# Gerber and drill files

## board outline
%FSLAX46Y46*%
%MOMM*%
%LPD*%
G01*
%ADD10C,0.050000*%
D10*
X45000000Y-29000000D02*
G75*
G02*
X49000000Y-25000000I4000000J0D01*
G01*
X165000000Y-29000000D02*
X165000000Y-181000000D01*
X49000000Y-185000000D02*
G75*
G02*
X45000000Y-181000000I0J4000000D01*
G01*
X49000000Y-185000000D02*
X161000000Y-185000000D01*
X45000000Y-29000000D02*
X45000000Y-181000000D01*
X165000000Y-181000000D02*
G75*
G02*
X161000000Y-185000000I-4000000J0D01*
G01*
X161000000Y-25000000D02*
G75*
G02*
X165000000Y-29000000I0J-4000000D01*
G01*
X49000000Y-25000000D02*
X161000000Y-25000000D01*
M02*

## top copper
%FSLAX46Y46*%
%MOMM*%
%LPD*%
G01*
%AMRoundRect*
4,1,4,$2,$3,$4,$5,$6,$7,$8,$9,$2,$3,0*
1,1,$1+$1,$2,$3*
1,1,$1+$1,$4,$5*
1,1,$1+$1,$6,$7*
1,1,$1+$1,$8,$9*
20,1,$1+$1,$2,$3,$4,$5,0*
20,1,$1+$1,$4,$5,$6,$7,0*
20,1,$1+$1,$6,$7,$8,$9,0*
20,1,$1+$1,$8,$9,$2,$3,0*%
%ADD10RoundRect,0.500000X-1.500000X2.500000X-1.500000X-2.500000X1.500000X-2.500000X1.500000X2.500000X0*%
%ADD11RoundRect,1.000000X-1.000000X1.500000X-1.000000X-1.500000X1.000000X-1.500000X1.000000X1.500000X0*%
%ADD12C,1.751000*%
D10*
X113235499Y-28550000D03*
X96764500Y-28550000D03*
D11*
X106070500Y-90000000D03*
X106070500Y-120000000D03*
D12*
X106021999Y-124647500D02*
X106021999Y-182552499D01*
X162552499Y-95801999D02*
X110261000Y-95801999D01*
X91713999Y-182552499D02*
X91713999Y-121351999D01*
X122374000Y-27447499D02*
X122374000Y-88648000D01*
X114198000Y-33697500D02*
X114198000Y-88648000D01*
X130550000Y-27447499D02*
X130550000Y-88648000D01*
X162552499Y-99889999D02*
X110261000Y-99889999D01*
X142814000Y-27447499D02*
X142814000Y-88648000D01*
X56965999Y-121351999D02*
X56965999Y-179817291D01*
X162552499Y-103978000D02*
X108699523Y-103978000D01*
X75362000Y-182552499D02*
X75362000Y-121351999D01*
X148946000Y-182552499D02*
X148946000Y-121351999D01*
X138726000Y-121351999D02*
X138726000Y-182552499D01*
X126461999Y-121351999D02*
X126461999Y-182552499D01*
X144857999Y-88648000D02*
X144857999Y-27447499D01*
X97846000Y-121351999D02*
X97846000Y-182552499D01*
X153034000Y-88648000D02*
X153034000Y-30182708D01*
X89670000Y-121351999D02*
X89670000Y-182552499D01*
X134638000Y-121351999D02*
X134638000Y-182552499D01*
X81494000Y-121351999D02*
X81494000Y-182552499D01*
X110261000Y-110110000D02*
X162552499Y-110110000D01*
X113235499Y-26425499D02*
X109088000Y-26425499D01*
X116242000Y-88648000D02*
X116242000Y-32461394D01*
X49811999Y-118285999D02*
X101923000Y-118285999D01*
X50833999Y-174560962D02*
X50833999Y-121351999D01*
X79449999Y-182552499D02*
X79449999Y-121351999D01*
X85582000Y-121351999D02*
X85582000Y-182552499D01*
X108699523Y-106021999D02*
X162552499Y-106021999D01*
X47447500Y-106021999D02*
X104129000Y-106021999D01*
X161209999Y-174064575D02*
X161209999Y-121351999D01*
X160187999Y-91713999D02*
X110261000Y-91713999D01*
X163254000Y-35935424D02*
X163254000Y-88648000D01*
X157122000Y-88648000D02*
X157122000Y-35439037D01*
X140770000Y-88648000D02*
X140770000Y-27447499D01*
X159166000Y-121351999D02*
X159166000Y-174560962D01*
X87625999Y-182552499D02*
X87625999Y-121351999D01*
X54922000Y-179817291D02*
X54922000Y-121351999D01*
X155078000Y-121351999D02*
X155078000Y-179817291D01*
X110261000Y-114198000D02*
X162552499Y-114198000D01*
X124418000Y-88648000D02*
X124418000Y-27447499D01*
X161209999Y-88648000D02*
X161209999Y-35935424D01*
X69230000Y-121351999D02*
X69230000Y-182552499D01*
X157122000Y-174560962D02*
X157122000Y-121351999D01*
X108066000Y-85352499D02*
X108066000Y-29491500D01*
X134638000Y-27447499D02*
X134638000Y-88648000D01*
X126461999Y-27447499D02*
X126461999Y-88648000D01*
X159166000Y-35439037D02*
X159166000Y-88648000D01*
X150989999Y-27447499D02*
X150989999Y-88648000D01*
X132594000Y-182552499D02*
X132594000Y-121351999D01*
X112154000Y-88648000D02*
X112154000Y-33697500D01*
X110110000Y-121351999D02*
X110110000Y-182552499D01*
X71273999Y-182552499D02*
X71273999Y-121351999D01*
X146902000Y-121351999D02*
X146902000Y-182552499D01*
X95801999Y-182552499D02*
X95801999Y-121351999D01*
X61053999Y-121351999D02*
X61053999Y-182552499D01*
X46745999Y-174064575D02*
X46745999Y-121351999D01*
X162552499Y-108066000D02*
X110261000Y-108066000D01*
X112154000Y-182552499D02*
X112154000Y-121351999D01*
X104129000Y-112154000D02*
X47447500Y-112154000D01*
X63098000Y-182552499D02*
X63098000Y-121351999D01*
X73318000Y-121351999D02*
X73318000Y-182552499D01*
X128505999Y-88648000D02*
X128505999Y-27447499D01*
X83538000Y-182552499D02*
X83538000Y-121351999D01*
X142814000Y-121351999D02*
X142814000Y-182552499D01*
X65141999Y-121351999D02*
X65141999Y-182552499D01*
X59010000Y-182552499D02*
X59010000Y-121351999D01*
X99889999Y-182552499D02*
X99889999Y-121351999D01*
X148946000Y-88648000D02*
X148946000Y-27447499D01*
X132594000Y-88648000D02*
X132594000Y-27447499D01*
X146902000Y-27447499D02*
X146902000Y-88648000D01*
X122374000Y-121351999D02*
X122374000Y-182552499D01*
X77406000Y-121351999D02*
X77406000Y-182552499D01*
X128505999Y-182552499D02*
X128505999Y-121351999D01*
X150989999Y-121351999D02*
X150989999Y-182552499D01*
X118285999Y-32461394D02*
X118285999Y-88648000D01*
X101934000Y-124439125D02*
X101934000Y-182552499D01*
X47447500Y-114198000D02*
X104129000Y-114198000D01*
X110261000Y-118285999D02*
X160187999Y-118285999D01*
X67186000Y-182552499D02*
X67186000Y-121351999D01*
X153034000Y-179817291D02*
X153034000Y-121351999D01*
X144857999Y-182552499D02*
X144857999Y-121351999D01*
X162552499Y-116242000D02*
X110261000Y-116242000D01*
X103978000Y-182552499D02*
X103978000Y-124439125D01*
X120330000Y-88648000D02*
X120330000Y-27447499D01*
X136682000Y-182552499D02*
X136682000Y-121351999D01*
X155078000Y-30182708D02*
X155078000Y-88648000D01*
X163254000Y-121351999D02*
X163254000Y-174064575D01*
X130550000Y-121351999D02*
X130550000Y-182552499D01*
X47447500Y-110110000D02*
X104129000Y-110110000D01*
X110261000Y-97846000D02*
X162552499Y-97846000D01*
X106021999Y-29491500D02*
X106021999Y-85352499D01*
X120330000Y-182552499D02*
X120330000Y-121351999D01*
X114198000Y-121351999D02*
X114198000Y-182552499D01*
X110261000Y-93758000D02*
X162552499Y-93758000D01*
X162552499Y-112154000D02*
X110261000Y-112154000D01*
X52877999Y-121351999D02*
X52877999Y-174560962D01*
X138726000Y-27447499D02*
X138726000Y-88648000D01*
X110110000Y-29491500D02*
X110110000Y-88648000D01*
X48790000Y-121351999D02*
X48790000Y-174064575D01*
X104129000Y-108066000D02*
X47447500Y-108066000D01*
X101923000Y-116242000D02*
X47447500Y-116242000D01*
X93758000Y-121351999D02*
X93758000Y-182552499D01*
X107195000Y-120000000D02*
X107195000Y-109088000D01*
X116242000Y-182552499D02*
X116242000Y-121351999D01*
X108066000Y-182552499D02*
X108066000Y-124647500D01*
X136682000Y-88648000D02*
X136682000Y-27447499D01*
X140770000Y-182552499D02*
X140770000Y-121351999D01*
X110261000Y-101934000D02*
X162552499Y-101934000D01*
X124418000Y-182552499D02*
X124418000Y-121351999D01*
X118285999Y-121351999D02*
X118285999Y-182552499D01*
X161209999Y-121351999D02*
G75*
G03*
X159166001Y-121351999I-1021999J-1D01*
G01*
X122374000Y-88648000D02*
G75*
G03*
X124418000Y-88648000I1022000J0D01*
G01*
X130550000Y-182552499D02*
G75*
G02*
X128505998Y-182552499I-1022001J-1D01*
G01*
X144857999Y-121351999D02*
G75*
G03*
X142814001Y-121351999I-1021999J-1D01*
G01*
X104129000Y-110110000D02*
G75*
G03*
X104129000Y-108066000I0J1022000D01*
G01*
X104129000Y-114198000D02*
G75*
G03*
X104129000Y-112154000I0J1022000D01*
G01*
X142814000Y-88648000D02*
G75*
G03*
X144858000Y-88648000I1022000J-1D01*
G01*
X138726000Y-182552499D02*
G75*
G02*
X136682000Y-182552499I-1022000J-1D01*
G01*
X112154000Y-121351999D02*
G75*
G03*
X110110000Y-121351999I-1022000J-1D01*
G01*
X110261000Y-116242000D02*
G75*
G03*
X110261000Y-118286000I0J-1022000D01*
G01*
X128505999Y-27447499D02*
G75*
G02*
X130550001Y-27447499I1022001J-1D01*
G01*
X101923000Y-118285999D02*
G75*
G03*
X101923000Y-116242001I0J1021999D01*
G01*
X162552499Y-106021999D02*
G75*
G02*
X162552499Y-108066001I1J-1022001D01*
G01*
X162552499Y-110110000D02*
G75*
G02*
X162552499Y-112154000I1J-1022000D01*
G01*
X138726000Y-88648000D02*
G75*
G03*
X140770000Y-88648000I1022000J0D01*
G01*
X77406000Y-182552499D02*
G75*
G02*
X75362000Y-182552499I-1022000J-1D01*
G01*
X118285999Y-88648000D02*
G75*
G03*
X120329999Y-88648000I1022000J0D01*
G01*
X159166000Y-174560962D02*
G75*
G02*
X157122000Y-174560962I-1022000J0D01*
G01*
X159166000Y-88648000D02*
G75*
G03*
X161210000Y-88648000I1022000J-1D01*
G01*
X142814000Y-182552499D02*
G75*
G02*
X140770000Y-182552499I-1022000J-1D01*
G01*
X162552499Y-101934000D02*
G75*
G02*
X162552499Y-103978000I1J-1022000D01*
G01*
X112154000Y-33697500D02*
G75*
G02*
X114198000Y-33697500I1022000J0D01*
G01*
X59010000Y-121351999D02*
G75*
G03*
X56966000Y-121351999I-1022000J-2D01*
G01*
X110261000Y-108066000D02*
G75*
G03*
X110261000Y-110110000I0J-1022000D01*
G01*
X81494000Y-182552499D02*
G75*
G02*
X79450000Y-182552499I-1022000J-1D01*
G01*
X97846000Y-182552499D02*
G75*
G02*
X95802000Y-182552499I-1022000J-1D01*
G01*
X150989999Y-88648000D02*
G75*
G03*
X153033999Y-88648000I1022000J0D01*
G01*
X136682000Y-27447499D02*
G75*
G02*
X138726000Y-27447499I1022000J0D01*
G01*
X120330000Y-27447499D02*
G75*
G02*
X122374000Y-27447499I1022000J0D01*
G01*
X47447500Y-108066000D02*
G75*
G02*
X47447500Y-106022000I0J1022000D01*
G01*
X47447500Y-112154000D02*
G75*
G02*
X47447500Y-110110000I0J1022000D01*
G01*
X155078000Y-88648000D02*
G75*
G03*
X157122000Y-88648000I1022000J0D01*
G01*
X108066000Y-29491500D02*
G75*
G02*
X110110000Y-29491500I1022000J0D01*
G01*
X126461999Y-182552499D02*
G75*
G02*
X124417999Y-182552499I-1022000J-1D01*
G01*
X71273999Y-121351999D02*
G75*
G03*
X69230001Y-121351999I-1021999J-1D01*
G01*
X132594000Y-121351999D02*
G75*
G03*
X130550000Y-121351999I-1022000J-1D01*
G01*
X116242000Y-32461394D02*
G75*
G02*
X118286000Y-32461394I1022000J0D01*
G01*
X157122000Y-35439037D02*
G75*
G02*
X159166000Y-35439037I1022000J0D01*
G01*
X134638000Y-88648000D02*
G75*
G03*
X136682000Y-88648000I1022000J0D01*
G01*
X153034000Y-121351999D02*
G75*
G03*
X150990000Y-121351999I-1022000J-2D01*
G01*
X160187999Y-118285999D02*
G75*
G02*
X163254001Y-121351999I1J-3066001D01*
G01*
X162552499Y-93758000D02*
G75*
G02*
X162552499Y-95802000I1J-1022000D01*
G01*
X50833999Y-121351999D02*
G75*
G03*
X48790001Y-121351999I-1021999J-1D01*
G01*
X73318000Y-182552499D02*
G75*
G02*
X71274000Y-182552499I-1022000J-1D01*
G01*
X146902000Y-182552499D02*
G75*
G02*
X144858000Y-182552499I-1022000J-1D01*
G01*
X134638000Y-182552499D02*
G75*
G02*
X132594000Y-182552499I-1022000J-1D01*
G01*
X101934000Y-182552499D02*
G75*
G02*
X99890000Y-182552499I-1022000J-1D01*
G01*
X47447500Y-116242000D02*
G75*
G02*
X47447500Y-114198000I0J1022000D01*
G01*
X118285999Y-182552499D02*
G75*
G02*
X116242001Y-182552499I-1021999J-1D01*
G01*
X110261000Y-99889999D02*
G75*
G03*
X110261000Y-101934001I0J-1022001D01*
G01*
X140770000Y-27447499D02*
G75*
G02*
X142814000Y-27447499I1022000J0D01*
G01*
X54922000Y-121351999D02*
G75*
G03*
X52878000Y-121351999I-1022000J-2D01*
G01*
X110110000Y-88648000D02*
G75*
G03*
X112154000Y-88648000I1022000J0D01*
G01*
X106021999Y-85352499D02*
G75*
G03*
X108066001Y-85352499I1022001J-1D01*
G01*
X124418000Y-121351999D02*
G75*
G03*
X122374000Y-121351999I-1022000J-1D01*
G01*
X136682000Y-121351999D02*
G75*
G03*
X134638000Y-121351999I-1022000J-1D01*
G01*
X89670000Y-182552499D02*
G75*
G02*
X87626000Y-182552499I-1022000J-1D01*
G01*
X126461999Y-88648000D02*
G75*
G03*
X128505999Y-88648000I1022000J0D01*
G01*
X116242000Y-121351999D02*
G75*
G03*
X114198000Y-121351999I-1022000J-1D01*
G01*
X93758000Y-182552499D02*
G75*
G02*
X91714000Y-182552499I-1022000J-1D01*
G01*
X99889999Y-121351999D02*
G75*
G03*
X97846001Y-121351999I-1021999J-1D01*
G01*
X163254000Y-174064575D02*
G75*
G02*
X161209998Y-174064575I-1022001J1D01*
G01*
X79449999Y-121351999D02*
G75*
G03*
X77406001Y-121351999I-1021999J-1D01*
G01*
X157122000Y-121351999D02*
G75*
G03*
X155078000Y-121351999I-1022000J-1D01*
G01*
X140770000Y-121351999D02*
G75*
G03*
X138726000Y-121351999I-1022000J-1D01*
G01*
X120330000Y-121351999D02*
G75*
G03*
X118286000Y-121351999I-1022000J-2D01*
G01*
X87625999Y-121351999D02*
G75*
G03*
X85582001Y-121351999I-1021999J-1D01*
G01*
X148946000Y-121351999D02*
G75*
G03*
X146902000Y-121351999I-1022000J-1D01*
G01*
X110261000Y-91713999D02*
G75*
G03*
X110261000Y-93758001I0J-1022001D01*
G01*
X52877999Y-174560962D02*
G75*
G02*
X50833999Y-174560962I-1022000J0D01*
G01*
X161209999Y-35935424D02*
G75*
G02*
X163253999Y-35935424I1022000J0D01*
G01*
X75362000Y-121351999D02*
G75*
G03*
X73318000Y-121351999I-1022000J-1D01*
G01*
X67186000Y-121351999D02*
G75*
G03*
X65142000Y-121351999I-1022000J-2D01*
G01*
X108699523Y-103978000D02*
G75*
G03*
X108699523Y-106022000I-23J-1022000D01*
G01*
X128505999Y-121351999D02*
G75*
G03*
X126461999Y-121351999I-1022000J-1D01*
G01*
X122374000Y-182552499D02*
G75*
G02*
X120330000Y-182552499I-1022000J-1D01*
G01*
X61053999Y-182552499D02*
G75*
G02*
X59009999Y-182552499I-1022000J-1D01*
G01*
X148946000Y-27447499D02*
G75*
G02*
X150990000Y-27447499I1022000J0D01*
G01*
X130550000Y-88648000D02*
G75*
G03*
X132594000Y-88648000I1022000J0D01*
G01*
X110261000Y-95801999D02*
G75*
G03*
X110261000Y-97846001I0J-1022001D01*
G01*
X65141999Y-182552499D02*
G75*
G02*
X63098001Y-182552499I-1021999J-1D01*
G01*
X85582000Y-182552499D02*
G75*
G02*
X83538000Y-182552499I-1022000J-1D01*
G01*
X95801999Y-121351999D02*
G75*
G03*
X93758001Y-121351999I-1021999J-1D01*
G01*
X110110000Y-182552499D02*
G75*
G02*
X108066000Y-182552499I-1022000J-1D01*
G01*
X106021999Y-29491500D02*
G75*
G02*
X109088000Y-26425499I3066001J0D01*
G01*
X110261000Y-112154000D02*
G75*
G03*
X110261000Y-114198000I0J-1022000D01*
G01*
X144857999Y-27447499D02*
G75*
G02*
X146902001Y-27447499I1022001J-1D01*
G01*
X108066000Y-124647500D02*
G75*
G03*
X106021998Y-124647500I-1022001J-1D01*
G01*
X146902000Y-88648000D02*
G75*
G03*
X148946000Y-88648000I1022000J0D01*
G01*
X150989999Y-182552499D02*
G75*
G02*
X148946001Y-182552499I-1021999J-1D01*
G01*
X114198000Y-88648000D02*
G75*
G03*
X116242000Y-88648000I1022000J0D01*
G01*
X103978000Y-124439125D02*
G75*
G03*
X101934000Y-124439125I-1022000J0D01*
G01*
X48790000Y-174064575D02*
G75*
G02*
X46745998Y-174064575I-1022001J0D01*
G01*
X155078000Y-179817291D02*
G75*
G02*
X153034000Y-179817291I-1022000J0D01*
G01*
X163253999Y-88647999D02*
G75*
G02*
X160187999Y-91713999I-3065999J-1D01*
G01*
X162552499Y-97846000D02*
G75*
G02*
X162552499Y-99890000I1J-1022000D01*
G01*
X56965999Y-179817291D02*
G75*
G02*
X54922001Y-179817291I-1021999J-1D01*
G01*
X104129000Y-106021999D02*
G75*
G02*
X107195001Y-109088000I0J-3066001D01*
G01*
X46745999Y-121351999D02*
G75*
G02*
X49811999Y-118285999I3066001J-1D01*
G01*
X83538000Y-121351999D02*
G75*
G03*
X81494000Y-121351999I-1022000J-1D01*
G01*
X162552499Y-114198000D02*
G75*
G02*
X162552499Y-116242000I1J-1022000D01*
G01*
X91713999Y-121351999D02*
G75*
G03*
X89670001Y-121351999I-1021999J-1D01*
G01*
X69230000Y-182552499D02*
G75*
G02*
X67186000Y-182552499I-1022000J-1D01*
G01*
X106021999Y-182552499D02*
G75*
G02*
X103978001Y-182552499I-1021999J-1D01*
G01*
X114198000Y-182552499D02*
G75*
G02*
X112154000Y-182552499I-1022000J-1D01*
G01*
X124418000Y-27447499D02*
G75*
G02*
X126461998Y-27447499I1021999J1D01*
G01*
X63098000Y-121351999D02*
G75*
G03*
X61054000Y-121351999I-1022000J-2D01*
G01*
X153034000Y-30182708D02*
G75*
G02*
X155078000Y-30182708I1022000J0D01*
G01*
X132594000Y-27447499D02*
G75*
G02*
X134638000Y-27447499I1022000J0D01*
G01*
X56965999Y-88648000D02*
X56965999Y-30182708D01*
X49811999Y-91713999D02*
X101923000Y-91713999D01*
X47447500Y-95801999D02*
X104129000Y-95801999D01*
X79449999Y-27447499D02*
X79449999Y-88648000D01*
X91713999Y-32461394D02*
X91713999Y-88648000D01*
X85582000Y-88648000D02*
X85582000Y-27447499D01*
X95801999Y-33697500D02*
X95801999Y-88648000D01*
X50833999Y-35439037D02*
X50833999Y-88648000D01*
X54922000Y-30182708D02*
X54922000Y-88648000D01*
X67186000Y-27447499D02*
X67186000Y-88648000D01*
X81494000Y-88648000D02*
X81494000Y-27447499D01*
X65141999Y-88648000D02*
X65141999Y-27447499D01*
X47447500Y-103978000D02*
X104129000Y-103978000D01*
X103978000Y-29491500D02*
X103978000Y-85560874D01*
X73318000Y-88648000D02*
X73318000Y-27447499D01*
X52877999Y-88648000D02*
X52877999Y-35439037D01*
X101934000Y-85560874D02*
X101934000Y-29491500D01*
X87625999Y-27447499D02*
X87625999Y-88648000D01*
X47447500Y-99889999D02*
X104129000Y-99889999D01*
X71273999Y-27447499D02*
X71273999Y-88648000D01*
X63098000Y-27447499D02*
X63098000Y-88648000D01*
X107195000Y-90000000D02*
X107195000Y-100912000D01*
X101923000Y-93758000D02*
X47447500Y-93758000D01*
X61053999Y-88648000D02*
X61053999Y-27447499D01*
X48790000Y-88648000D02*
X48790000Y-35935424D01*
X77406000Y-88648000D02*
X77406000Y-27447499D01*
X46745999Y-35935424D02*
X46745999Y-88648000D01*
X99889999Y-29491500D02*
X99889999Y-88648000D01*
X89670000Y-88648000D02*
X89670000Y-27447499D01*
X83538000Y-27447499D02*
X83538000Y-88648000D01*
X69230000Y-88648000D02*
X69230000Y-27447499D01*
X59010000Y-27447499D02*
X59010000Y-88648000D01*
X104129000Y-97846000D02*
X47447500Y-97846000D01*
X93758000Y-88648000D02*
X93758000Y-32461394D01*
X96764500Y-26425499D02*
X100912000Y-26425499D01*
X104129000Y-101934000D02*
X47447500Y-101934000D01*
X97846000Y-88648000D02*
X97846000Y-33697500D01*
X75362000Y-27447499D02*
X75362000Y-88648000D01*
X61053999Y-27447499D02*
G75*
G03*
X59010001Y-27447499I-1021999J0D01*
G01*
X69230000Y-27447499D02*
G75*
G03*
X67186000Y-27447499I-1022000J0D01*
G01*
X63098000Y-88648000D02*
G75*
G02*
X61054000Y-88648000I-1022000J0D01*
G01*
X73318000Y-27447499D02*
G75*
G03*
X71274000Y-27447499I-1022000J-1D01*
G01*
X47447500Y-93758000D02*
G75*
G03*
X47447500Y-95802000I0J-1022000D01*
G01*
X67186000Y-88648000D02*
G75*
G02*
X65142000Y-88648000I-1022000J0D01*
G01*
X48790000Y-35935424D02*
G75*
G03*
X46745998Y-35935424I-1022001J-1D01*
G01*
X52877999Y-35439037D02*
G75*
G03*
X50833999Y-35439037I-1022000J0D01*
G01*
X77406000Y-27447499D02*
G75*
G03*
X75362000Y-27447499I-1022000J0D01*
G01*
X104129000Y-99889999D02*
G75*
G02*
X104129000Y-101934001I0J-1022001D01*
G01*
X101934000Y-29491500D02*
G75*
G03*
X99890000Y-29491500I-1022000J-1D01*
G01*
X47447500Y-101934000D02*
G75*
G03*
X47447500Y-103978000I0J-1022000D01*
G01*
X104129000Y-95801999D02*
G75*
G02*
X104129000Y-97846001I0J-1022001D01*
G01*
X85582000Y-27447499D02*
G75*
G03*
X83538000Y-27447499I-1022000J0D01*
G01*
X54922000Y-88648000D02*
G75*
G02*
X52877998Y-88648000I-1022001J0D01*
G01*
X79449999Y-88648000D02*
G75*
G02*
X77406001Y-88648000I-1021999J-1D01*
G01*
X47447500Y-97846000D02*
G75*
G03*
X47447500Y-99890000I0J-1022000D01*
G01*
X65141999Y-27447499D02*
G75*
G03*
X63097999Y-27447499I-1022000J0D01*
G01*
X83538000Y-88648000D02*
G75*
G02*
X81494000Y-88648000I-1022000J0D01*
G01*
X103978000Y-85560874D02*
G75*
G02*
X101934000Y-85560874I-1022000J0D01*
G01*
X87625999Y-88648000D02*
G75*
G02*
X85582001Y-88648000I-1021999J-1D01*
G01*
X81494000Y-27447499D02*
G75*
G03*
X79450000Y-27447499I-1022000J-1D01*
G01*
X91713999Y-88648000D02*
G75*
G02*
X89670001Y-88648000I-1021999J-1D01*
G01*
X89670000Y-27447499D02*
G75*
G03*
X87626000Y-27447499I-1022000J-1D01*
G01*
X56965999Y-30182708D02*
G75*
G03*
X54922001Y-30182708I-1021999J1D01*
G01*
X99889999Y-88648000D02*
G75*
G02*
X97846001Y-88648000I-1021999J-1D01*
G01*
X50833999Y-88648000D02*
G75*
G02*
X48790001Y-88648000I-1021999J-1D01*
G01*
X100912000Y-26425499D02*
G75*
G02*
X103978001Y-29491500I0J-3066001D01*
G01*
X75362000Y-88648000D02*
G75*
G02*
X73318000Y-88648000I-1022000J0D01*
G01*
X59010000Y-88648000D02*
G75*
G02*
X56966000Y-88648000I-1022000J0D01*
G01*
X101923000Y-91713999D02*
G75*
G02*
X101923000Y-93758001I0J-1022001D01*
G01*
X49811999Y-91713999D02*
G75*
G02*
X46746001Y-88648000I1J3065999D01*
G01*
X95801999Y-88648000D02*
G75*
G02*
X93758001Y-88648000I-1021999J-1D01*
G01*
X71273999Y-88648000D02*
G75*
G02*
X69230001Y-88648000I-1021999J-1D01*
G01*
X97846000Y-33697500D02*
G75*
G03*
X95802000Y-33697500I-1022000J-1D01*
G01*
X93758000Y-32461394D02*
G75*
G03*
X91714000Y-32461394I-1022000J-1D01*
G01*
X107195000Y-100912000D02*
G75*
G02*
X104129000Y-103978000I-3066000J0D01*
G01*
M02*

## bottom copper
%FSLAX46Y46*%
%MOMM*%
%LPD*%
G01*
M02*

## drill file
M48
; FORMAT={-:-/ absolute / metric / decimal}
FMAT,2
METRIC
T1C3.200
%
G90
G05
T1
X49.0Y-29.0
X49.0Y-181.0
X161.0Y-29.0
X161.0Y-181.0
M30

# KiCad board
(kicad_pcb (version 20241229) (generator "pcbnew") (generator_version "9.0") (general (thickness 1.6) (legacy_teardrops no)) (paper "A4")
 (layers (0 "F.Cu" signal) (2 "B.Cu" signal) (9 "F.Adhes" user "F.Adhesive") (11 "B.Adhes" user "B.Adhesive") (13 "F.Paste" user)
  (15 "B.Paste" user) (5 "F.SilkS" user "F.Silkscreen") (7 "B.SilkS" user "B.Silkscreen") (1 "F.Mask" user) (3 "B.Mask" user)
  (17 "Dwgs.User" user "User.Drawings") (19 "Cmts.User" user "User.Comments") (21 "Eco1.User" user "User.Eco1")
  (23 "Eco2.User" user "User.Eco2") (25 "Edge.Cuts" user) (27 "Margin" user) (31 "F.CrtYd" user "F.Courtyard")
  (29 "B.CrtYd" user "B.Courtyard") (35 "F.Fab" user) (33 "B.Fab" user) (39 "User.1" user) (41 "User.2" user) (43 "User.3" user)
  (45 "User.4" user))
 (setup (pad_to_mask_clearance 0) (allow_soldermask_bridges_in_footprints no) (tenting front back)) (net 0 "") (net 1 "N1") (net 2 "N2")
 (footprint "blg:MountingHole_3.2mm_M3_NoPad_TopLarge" (layer "F.Cu") (at 161 29)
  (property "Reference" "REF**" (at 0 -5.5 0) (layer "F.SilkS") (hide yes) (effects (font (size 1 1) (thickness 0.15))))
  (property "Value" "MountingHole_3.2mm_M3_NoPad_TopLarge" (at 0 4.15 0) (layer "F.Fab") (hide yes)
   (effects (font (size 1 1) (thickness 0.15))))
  (pad "" np_thru_hole circle (at 0 0) (size 7.6 7.6) (drill 3.2) (layers) (zone_connect 2)))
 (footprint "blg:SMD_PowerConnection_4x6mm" (layer "F.Cu") (at 113.235499 28.55 -90)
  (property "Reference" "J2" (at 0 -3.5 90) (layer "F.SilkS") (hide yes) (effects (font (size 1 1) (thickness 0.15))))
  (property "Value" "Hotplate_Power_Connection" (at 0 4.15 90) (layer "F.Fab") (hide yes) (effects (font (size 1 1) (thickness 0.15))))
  (pad "1" smd roundrect (at 0 0 270) (size 6 4) (layers "F.Cu" "F.Mask" "F.Paste") (roundrect_rratio 0.125) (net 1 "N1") (zone_connect 2)))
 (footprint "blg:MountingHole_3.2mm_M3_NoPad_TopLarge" (layer "F.Cu") (at 49 181)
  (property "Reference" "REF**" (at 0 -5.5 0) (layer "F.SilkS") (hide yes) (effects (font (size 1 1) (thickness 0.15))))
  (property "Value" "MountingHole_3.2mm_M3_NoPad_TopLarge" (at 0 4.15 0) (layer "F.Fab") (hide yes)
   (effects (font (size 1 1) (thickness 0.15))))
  (pad "" np_thru_hole circle (at 0 0) (size 7.6 7.6) (drill 3.2) (layers) (zone_connect 2)))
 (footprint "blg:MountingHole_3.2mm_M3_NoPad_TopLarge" (layer "F.Cu") (at 161 181)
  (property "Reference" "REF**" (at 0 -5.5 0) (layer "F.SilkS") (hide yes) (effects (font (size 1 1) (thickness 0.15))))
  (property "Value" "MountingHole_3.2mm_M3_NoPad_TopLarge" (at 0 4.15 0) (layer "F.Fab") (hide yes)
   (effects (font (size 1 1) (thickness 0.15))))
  (pad "" np_thru_hole circle (at 0 0) (size 7.6 7.6) (drill 3.2) (layers) (zone_connect 2)))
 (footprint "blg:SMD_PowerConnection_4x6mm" (layer "F.Cu") (at 96.7645 28.55 -90)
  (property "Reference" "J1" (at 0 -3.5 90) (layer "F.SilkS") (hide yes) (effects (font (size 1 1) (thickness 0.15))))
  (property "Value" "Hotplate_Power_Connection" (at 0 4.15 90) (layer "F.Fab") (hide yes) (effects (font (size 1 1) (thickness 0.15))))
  (pad "1" smd roundrect (at 0 0 270) (size 6 4) (layers "F.Cu" "F.Mask" "F.Paste") (roundrect_rratio 0.125) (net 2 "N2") (zone_connect 2)))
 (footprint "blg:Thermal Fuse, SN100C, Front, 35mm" (layer "F.Cu") (at 106.0705 105 -90)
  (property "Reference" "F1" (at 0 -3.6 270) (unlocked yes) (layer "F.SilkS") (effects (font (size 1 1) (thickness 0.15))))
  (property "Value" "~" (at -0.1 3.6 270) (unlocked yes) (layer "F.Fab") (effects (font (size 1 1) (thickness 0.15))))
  (pad "1" smd roundrect (at -15 0 270) (size 5 4) (layers "F.Cu" "F.Mask") (roundrect_rratio 0.25) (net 2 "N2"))
  (pad "2" smd roundrect (at 15 0 270) (size 5 4) (layers "F.Cu" "F.Mask") (roundrect_rratio 0.25) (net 1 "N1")))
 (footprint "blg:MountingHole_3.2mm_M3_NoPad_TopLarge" (layer "F.Cu") (at 49 29)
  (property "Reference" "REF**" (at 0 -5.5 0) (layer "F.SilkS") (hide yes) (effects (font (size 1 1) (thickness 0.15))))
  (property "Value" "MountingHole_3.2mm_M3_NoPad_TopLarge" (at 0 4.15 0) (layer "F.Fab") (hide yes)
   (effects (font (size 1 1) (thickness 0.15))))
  (pad "" np_thru_hole circle (at 0 0) (size 7.6 7.6) (drill 3.2) (layers) (zone_connect 2)))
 (gr_arc (start 45 29) (mid 46.171573 26.171573) (end 49 25) (stroke (width 0.05) (type solid)) (layer "Edge.Cuts"))
 (gr_line (start 165 29) (end 165 181) (stroke (width 0.05) (type default)) (layer "Edge.Cuts"))
 (gr_arc (start 49 185) (mid 46.171573 183.828427) (end 45 181) (stroke (width 0.05) (type solid)) (layer "Edge.Cuts"))
 (gr_line (start 49 185) (end 161 185) (stroke (width 0.05) (type default)) (layer "Edge.Cuts"))
 (gr_line (start 45 29) (end 45 181) (stroke (width 0.05) (type default)) (layer "Edge.Cuts"))
 (gr_arc (start 165 181) (mid 163.828427 183.828427) (end 161 185) (stroke (width 0.05) (type solid)) (layer "Edge.Cuts"))
 (gr_arc (start 161 25) (mid 163.828427 26.171573) (end 165 29) (stroke (width 0.05) (type solid)) (layer "Edge.Cuts"))
 (gr_line (start 49 25) (end 161 25) (stroke (width 0.05) (type default)) (layer "Edge.Cuts"))
 (segment (start 106.021999 124.6475) (end 106.021999 182.552499) (width 1.751) (layer "F.Cu") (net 1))
 (segment (start 162.552499 95.801999) (end 110.261 95.801999) (width 1.751) (layer "F.Cu") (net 1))
 (segment (start 91.713999 182.552499) (end 91.713999 121.351999) (width 1.751) (layer "F.Cu") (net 1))
 (segment (start 122.374 27.447499) (end 122.374 88.648) (width 1.751) (layer "F.Cu") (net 1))
 (segment (start 114.198 33.6975) (end 114.198 88.648) (width 1.751) (layer "F.Cu") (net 1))
 (segment (start 130.55 27.447499) (end 130.55 88.648) (width 1.751) (layer "F.Cu") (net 1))
 (segment (start 162.552499 99.889999) (end 110.261 99.889999) (width 1.751) (layer "F.Cu") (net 1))
 (segment (start 142.814 27.447499) (end 142.814 88.648) (width 1.751) (layer "F.Cu") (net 1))
 (segment (start 56.965999 121.351999) (end 56.965999 179.817291) (width 1.751) (layer "F.Cu") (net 1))
 (segment (start 162.552499 103.978) (end 108.699523 103.978) (width 1.751) (layer "F.Cu") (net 1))
 (segment (start 75.362 182.552499) (end 75.362 121.351999) (width 1.751) (layer "F.Cu") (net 1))
 (segment (start 148.946 182.552499) (end 148.946 121.351999) (width 1.751) (layer "F.Cu") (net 1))
 (segment (start 138.726 121.351999) (end 138.726 182.552499) (width 1.751) (layer "F.Cu") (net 1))
 (segment (start 126.461999 121.351999) (end 126.461999 182.552499) (width 1.751) (layer "F.Cu") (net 1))
 (segment (start 144.857999 88.648) (end 144.857999 27.447499) (width 1.751) (layer "F.Cu") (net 1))
 (segment (start 97.846 121.351999) (end 97.846 182.552499) (width 1.751) (layer "F.Cu") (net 1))
 (segment (start 153.034 88.648) (end 153.034 30.182708) (width 1.751) (layer "F.Cu") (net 1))
 (segment (start 89.67 121.351999) (end 89.67 182.552499) (width 1.751) (layer "F.Cu") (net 1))
 (segment (start 134.638 121.351999) (end 134.638 182.552499) (width 1.751) (layer "F.Cu") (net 1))
 (segment (start 81.494 121.351999) (end 81.494 182.552499) (width 1.751) (layer "F.Cu") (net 1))
 (segment (start 110.261 110.11) (end 162.552499 110.11) (width 1.751) (layer "F.Cu") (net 1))
 (segment (start 113.235499 26.425499) (end 109.088 26.425499) (width 1.751) (layer "F.Cu") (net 1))
 (segment (start 116.242 88.648) (end 116.242 32.461394) (width 1.751) (layer "F.Cu") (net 1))
 (segment (start 49.811999 118.285999) (end 101.923 118.285999) (width 1.751) (layer "F.Cu") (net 1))
 (segment (start 50.833999 174.560962) (end 50.833999 121.351999) (width 1.751) (layer "F.Cu") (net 1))
 (segment (start 79.449999 182.552499) (end 79.449999 121.351999) (width 1.751) (layer "F.Cu") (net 1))
 (segment (start 85.582 121.351999) (end 85.582 182.552499) (width 1.751) (layer "F.Cu") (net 1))
 (segment (start 108.699523 106.021999) (end 162.552499 106.021999) (width 1.751) (layer "F.Cu") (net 1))
 (segment (start 47.4475 106.021999) (end 104.129 106.021999) (width 1.751) (layer "F.Cu") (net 1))
 (segment (start 161.209999 174.064575) (end 161.209999 121.351999) (width 1.751) (layer "F.Cu") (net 1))
 (segment (start 160.187999 91.713999) (end 110.261 91.713999) (width 1.751) (layer "F.Cu") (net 1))
 (segment (start 163.254 35.935424) (end 163.254 88.648) (width 1.751) (layer "F.Cu") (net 1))
 (segment (start 157.122 88.648) (end 157.122 35.439037) (width 1.751) (layer "F.Cu") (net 1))
 (segment (start 140.77 88.648) (end 140.77 27.447499) (width 1.751) (layer "F.Cu") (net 1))
 (segment (start 159.166 121.351999) (end 159.166 174.560962) (width 1.751) (layer "F.Cu") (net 1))
 (segment (start 87.625999 182.552499) (end 87.625999 121.351999) (width 1.751) (layer "F.Cu") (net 1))
 (segment (start 54.922 179.817291) (end 54.922 121.351999) (width 1.751) (layer "F.Cu") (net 1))
 (segment (start 155.078 121.351999) (end 155.078 179.817291) (width 1.751) (layer "F.Cu") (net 1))
 (segment (start 110.261 114.198) (end 162.552499 114.198) (width 1.751) (layer "F.Cu") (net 1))
 (segment (start 124.418 88.648) (end 124.418 27.447499) (width 1.751) (layer "F.Cu") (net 1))
 (segment (start 161.209999 88.648) (end 161.209999 35.935424) (width 1.751) (layer "F.Cu") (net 1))
 (segment (start 69.23 121.351999) (end 69.23 182.552499) (width 1.751) (layer "F.Cu") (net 1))
 (segment (start 157.122 174.560962) (end 157.122 121.351999) (width 1.751) (layer "F.Cu") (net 1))
 (segment (start 108.066 85.352499) (end 108.066 29.4915) (width 1.751) (layer "F.Cu") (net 1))
 (segment (start 134.638 27.447499) (end 134.638 88.648) (width 1.751) (layer "F.Cu") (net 1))
 (segment (start 126.461999 27.447499) (end 126.461999 88.648) (width 1.751) (layer "F.Cu") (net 1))
 (segment (start 159.166 35.439037) (end 159.166 88.648) (width 1.751) (layer "F.Cu") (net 1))
 (segment (start 150.989999 27.447499) (end 150.989999 88.648) (width 1.751) (layer "F.Cu") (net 1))
 (segment (start 132.594 182.552499) (end 132.594 121.351999) (width 1.751) (layer "F.Cu") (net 1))
 (segment (start 112.154 88.648) (end 112.154 33.6975) (width 1.751) (layer "F.Cu") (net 1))
 (segment (start 110.11 121.351999) (end 110.11 182.552499) (width 1.751) (layer "F.Cu") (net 1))
 (segment (start 71.273999 182.552499) (end 71.273999 121.351999) (width 1.751) (layer "F.Cu") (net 1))
 (segment (start 146.902 121.351999) (end 146.902 182.552499) (width 1.751) (layer "F.Cu") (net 1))
 (segment (start 95.801999 182.552499) (end 95.801999 121.351999) (width 1.751) (layer "F.Cu") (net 1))
 (segment (start 61.053999 121.351999) (end 61.053999 182.552499) (width 1.751) (layer "F.Cu") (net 1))
 (segment (start 46.745999 174.064575) (end 46.745999 121.351999) (width 1.751) (layer "F.Cu") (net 1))
 (segment (start 162.552499 108.066) (end 110.261 108.066) (width 1.751) (layer "F.Cu") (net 1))
 (segment (start 112.154 182.552499) (end 112.154 121.351999) (width 1.751) (layer "F.Cu") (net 1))
 (segment (start 104.129 112.154) (end 47.4475 112.154) (width 1.751) (layer "F.Cu") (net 1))
 (segment (start 63.098 182.552499) (end 63.098 121.351999) (width 1.751) (layer "F.Cu") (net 1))
 (segment (start 73.318 121.351999) (end 73.318 182.552499) (width 1.751) (layer "F.Cu") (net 1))
 (segment (start 128.505999 88.648) (end 128.505999 27.447499) (width 1.751) (layer "F.Cu") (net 1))
 (segment (start 83.538 182.552499) (end 83.538 121.351999) (width 1.751) (layer "F.Cu") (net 1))
 (segment (start 142.814 121.351999) (end 142.814 182.552499) (width 1.751) (layer "F.Cu") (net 1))
 (segment (start 65.141999 121.351999) (end 65.141999 182.552499) (width 1.751) (layer "F.Cu") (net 1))
 (segment (start 59.01 182.552499) (end 59.01 121.351999) (width 1.751) (layer "F.Cu") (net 1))
 (segment (start 99.889999 182.552499) (end 99.889999 121.351999) (width 1.751) (layer "F.Cu") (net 1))
 (segment (start 148.946 88.648) (end 148.946 27.447499) (width 1.751) (layer "F.Cu") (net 1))
 (segment (start 132.594 88.648) (end 132.594 27.447499) (width 1.751) (layer "F.Cu") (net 1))
 (segment (start 146.902 27.447499) (end 146.902 88.648) (width 1.751) (layer "F.Cu") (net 1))
 (segment (start 122.374 121.351999) (end 122.374 182.552499) (width 1.751) (layer "F.Cu") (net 1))
 (segment (start 77.406 121.351999) (end 77.406 182.552499) (width 1.751) (layer "F.Cu") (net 1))
 (segment (start 128.505999 182.552499) (end 128.505999 121.351999) (width 1.751) (layer "F.Cu") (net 1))
 (segment (start 150.989999 121.351999) (end 150.989999 182.552499) (width 1.751) (layer "F.Cu") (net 1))
 (segment (start 118.285999 32.461394) (end 118.285999 88.648) (width 1.751) (layer "F.Cu") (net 1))
 (segment (start 101.934 124.439125) (end 101.934 182.552499) (width 1.751) (layer "F.Cu") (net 1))
 (segment (start 47.4475 114.198) (end 104.129 114.198) (width 1.751) (layer "F.Cu") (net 1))
 (segment (start 110.261 118.285999) (end 160.187999 118.285999) (width 1.751) (layer "F.Cu") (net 1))
 (segment (start 67.186 182.552499) (end 67.186 121.351999) (width 1.751) (layer "F.Cu") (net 1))
 (segment (start 153.034 179.817291) (end 153.034 121.351999) (width 1.751) (layer "F.Cu") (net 1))
 (segment (start 144.857999 182.552499) (end 144.857999 121.351999) (width 1.751) (layer "F.Cu") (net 1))
 (segment (start 162.552499 116.242) (end 110.261 116.242) (width 1.751) (layer "F.Cu") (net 1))
 (segment (start 103.978 182.552499) (end 103.978 124.439125) (width 1.751) (layer "F.Cu") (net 1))
 (segment (start 120.33 88.648) (end 120.33 27.447499) (width 1.751) (layer "F.Cu") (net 1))
 (segment (start 136.682 182.552499) (end 136.682 121.351999) (width 1.751) (layer "F.Cu") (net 1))
 (segment (start 155.078 30.182708) (end 155.078 88.648) (width 1.751) (layer "F.Cu") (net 1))
 (segment (start 163.254 121.351999) (end 163.254 174.064575) (width 1.751) (layer "F.Cu") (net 1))
 (segment (start 130.55 121.351999) (end 130.55 182.552499) (width 1.751) (layer "F.Cu") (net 1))
 (segment (start 47.4475 110.11) (end 104.129 110.11) (width 1.751) (layer "F.Cu") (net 1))
 (segment (start 110.261 97.846) (end 162.552499 97.846) (width 1.751) (layer "F.Cu") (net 1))
 (segment (start 106.021999 29.4915) (end 106.021999 85.352499) (width 1.751) (layer "F.Cu") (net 1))
 (segment (start 120.33 182.552499) (end 120.33 121.351999) (width 1.751) (layer "F.Cu") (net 1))
 (segment (start 114.198 121.351999) (end 114.198 182.552499) (width 1.751) (layer "F.Cu") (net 1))
 (segment (start 110.261 93.758) (end 162.552499 93.758) (width 1.751) (layer "F.Cu") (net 1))
 (segment (start 162.552499 112.154) (end 110.261 112.154) (width 1.751) (layer "F.Cu") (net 1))
 (segment (start 52.877999 121.351999) (end 52.877999 174.560962) (width 1.751) (layer "F.Cu") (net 1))
 (segment (start 138.726 27.447499) (end 138.726 88.648) (width 1.751) (layer "F.Cu") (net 1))
 (segment (start 110.11 29.4915) (end 110.11 88.648) (width 1.751) (layer "F.Cu") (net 1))
 (segment (start 48.79 121.351999) (end 48.79 174.064575) (width 1.751) (layer "F.Cu") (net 1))
 (segment (start 104.129 108.066) (end 47.4475 108.066) (width 1.751) (layer "F.Cu") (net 1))
 (segment (start 101.923 116.242) (end 47.4475 116.242) (width 1.751) (layer "F.Cu") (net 1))
 (segment (start 93.758 121.351999) (end 93.758 182.552499) (width 1.751) (layer "F.Cu") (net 1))
 (segment (start 107.195 120) (end 107.195 109.088) (width 1.751) (layer "F.Cu") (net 1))
 (segment (start 116.242 182.552499) (end 116.242 121.351999) (width 1.751) (layer "F.Cu") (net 1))
 (segment (start 108.066 182.552499) (end 108.066 124.6475) (width 1.751) (layer "F.Cu") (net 1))
 (segment (start 136.682 88.648) (end 136.682 27.447499) (width 1.751) (layer "F.Cu") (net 1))
 (segment (start 140.77 182.552499) (end 140.77 121.351999) (width 1.751) (layer "F.Cu") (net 1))
 (segment (start 110.261 101.934) (end 162.552499 101.934) (width 1.751) (layer "F.Cu") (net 1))
 (segment (start 124.418 182.552499) (end 124.418 121.351999) (width 1.751) (layer "F.Cu") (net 1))
 (segment (start 118.285999 121.351999) (end 118.285999 182.552499) (width 1.751) (layer "F.Cu") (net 1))
 (arc (start 161.209999 121.351999) (mid 160.188 120.33) (end 159.166 121.351999) (width 1.751) (layer "F.Cu") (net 1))
 (arc (start 122.374 88.648) (mid 123.395999 89.67) (end 124.418 88.648) (width 1.751) (layer "F.Cu") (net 1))
 (arc (start 130.55 182.552499) (mid 129.527999 183.5745) (end 128.505999 182.552499) (width 1.751) (layer "F.Cu") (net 1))
 (arc (start 144.857999 121.351999) (mid 143.835999 120.33) (end 142.814 121.351999) (width 1.751) (layer "F.Cu") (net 1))
 (arc (start 104.129 110.11) (mid 105.151 109.088) (end 104.129 108.066) (width 1.751) (layer "F.Cu") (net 1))
 (arc (start 104.129 114.198) (mid 105.151 113.176) (end 104.129 112.154) (width 1.751) (layer "F.Cu") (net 1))
 (arc (start 142.814 88.648) (mid 143.835999 89.67) (end 144.857999 88.648) (width 1.751) (layer "F.Cu") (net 1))
 (arc (start 138.726 182.552499) (mid 137.703999 183.5745) (end 136.682 182.552499) (width 1.751) (layer "F.Cu") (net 1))
 (arc (start 112.154 121.351999) (mid 111.131999 120.33) (end 110.11 121.351999) (width 1.751) (layer "F.Cu") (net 1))
 (arc (start 110.261 116.242) (mid 109.238999 117.264) (end 110.261 118.285999) (width 1.751) (layer "F.Cu") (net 1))
 (arc (start 128.505999 27.447499) (mid 129.527999 26.425499) (end 130.55 27.447499) (width 1.751) (layer "F.Cu") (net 1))
 (arc (start 101.923 118.285999) (mid 102.945 117.264) (end 101.923 116.242) (width 1.751) (layer "F.Cu") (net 1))
 (arc (start 162.552499 106.021999) (mid 163.574499 107.044) (end 162.552499 108.066) (width 1.751) (layer "F.Cu") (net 1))
 (arc (start 162.552499 110.11) (mid 163.574499 111.131999) (end 162.552499 112.154) (width 1.751) (layer "F.Cu") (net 1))
 (arc (start 138.726 88.648) (mid 139.748 89.67) (end 140.77 88.648) (width 1.751) (layer "F.Cu") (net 1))
 (arc (start 77.406 182.552499) (mid 76.384 183.5745) (end 75.362 182.552499) (width 1.751) (layer "F.Cu") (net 1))
 (arc (start 118.285999 88.648) (mid 119.308 89.67) (end 120.33 88.648) (width 1.751) (layer "F.Cu") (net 1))
 (arc (start 159.166 174.560962) (mid 158.143999 175.582962) (end 157.122 174.560962) (width 1.751) (layer "F.Cu") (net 1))
 (arc (start 159.166 88.648) (mid 160.188 89.67) (end 161.209999 88.648) (width 1.751) (layer "F.Cu") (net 1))
 (arc (start 142.814 182.552499) (mid 141.792 183.5745) (end 140.77 182.552499) (width 1.751) (layer "F.Cu") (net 1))
 (arc (start 162.552499 101.934) (mid 163.574499 102.955999) (end 162.552499 103.978) (width 1.751) (layer "F.Cu") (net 1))
 (arc (start 112.154 33.6975) (mid 113.176 32.6755) (end 114.198 33.6975) (width 1.751) (layer "F.Cu") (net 1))
 (arc (start 59.01 121.351999) (mid 57.988 120.33) (end 56.965999 121.351999) (width 1.751) (layer "F.Cu") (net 1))
 (arc (start 110.261 108.066) (mid 109.238999 109.088) (end 110.261 110.11) (width 1.751) (layer "F.Cu") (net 1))
 (arc (start 81.494 182.552499) (mid 80.472 183.5745) (end 79.449999 182.552499) (width 1.751) (layer "F.Cu") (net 1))
 (arc (start 97.846 182.552499) (mid 96.824 183.5745) (end 95.801999 182.552499) (width 1.751) (layer "F.Cu") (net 1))
 (arc (start 150.989999 88.648) (mid 152.011999 89.67) (end 153.034 88.648) (width 1.751) (layer "F.Cu") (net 1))
 (arc (start 136.682 27.447499) (mid 137.703999 26.425499) (end 138.726 27.447499) (width 1.751) (layer "F.Cu") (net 1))
 (arc (start 120.33 27.447499) (mid 121.351999 26.425499) (end 122.374 27.447499) (width 1.751) (layer "F.Cu") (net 1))
 (arc (start 47.4475 108.066) (mid 46.425499 107.044) (end 47.4475 106.021999) (width 1.751) (layer "F.Cu") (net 1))
 (arc (start 47.4475 112.154) (mid 46.425499 111.131999) (end 47.4475 110.11) (width 1.751) (layer "F.Cu") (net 1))
 (arc (start 155.078 88.648) (mid 156.1 89.67) (end 157.122 88.648) (width 1.751) (layer "F.Cu") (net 1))
 (arc (start 108.066 29.4915) (mid 109.088 28.4695) (end 110.11 29.4915) (width 1.751) (layer "F.Cu") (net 1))
 (arc (start 126.461999 182.552499) (mid 125.44 183.5745) (end 124.418 182.552499) (width 1.751) (layer "F.Cu") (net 1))
 (arc (start 71.273999 121.351999) (mid 70.252 120.33) (end 69.23 121.351999) (width 1.751) (layer "F.Cu") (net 1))
 (arc (start 132.594 121.351999) (mid 131.572 120.33) (end 130.55 121.351999) (width 1.751) (layer "F.Cu") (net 1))
 (arc (start 116.242 32.461394) (mid 117.264 31.439394) (end 118.285999 32.461394) (width 1.751) (layer "F.Cu") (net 1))
 (arc (start 157.122 35.439037) (mid 158.143999 34.417037) (end 159.166 35.439037) (width 1.751) (layer "F.Cu") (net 1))
 (arc (start 134.638 88.648) (mid 135.66 89.67) (end 136.682 88.648) (width 1.751) (layer "F.Cu") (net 1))
 (arc (start 153.034 121.351999) (mid 152.011999 120.33) (end 150.989999 121.351999) (width 1.751) (layer "F.Cu") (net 1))
 (arc (start 160.187999 118.285999) (mid 162.355989 119.18401) (end 163.253999 121.351999) (width 1.751) (layer "F.Cu") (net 1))
 (arc (start 162.552499 93.758) (mid 163.574499 94.779999) (end 162.552499 95.801999) (width 1.751) (layer "F.Cu") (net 1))
 (arc (start 50.833999 121.351999) (mid 49.812 120.33) (end 48.79 121.351999) (width 1.751) (layer "F.Cu") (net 1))
 (arc (start 73.318 182.552499) (mid 72.295999 183.5745) (end 71.273999 182.552499) (width 1.751) (layer "F.Cu") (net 1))
 (arc (start 146.902 182.552499) (mid 145.88 183.5745) (end 144.857999 182.552499) (width 1.751) (layer "F.Cu") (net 1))
 (arc (start 134.638 182.552499) (mid 133.615999 183.5745) (end 132.594 182.552499) (width 1.751) (layer "F.Cu") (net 1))
 (arc (start 101.934 182.552499) (mid 100.912 183.5745) (end 99.889999 182.552499) (width 1.751) (layer "F.Cu") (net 1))
 (arc (start 47.4475 116.242) (mid 46.425499 115.219999) (end 47.4475 114.198) (width 1.751) (layer "F.Cu") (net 1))
 (arc (start 118.285999 182.552499) (mid 117.264 183.5745) (end 116.242 182.552499) (width 1.751) (layer "F.Cu") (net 1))
 (arc (start 110.261 99.889999) (mid 109.238999 100.912) (end 110.261 101.934) (width 1.751) (layer "F.Cu") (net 1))
 (arc (start 140.77 27.447499) (mid 141.792 26.425499) (end 142.814 27.447499) (width 1.751) (layer "F.Cu") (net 1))
 (arc (start 54.922 121.351999) (mid 53.9 120.33) (end 52.877999 121.351999) (width 1.751) (layer "F.Cu") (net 1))
 (arc (start 110.11 88.648) (mid 111.131999 89.67) (end 112.154 88.648) (width 1.751) (layer "F.Cu") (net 1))
 (arc (start 106.021999 85.352499) (mid 107.044 86.3745) (end 108.066 85.352499) (width 1.751) (layer "F.Cu") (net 1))
 (arc (start 124.418 121.351999) (mid 123.395999 120.33) (end 122.374 121.351999) (width 1.751) (layer "F.Cu") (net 1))
 (arc (start 136.682 121.351999) (mid 135.66 120.33) (end 134.638 121.351999) (width 1.751) (layer "F.Cu") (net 1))
 (arc (start 89.67 182.552499) (mid 88.648 183.5745) (end 87.625999 182.552499) (width 1.751) (layer "F.Cu") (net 1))
 (arc (start 126.461999 88.648) (mid 127.483999 89.67) (end 128.505999 88.648) (width 1.751) (layer "F.Cu") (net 1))
 (arc (start 116.242 121.351999) (mid 115.219999 120.33) (end 114.198 121.351999) (width 1.751) (layer "F.Cu") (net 1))
 (arc (start 93.758 182.552499) (mid 92.736 183.5745) (end 91.713999 182.552499) (width 1.751) (layer "F.Cu") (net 1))
 (arc (start 99.889999 121.351999) (mid 98.868 120.33) (end 97.846 121.351999) (width 1.751) (layer "F.Cu") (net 1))
 (arc (start 163.254 174.064575) (mid 162.232 175.086575) (end 161.209999 174.064575) (width 1.751) (layer "F.Cu") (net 1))
 (arc (start 79.449999 121.351999) (mid 78.428 120.33) (end 77.406 121.351999) (width 1.751) (layer "F.Cu") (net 1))
 (arc (start 157.122 121.351999) (mid 156.1 120.33) (end 155.078 121.351999) (width 1.751) (layer "F.Cu") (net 1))
 (arc (start 140.77 121.351999) (mid 139.748 120.33) (end 138.726 121.351999) (width 1.751) (layer "F.Cu") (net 1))
 (arc (start 120.33 121.351999) (mid 119.308 120.33) (end 118.285999 121.351999) (width 1.751) (layer "F.Cu") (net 1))
 (arc (start 87.625999 121.351999) (mid 86.604 120.33) (end 85.582 121.351999) (width 1.751) (layer "F.Cu") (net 1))
 (arc (start 148.946 121.351999) (mid 147.924 120.33) (end 146.902 121.351999) (width 1.751) (layer "F.Cu") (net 1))
 (arc (start 110.261 91.713999) (mid 109.238999 92.736) (end 110.261 93.758) (width 1.751) (layer "F.Cu") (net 1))
 (arc (start 52.877999 174.560962) (mid 51.856 175.582962) (end 50.833999 174.560962) (width 1.751) (layer "F.Cu") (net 1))
 (arc (start 161.209999 35.935424) (mid 162.232 34.913424) (end 163.254 35.935424) (width 1.751) (layer "F.Cu") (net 1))
 (arc (start 75.362 121.351999) (mid 74.34 120.33) (end 73.318 121.351999) (width 1.751) (layer "F.Cu") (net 1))
 (arc (start 67.186 121.351999) (mid 66.164 120.33) (end 65.141999 121.351999) (width 1.751) (layer "F.Cu") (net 1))
 (arc (start 108.699523 103.978) (mid 107.677523 105) (end 108.699523 106.021999) (width 1.751) (layer "F.Cu") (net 1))
 (arc (start 128.505999 121.351999) (mid 127.483999 120.33) (end 126.461999 121.351999) (width 1.751) (layer "F.Cu") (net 1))
 (arc (start 122.374 182.552499) (mid 121.351999 183.5745) (end 120.33 182.552499) (width 1.751) (layer "F.Cu") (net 1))
 (arc (start 61.053999 182.552499) (mid 60.032 183.5745) (end 59.01 182.552499) (width 1.751) (layer "F.Cu") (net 1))
 (arc (start 148.946 27.447499) (mid 149.968 26.425499) (end 150.989999 27.447499) (width 1.751) (layer "F.Cu") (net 1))
 (arc (start 130.55 88.648) (mid 131.572 89.67) (end 132.594 88.648) (width 1.751) (layer "F.Cu") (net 1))
 (arc (start 110.261 95.801999) (mid 109.238999 96.824) (end 110.261 97.846) (width 1.751) (layer "F.Cu") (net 1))
 (arc (start 65.141999 182.552499) (mid 64.119999 183.5745) (end 63.098 182.552499) (width 1.751) (layer "F.Cu") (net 1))
 (arc (start 85.582 182.552499) (mid 84.56 183.5745) (end 83.538 182.552499) (width 1.751) (layer "F.Cu") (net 1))
 (arc (start 95.801999 121.351999) (mid 94.779999 120.33) (end 93.758 121.351999) (width 1.751) (layer "F.Cu") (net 1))
 (arc (start 110.11 182.552499) (mid 109.088 183.5745) (end 108.066 182.552499) (width 1.751) (layer "F.Cu") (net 1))
 (arc (start 106.021999 29.4915) (mid 106.92001 27.32351) (end 109.088 26.425499) (width 1.751) (layer "F.Cu") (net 1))
 (arc (start 110.261 112.154) (mid 109.238999 113.176) (end 110.261 114.198) (width 1.751) (layer "F.Cu") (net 1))
 (arc (start 144.857999 27.447499) (mid 145.88 26.425499) (end 146.902 27.447499) (width 1.751) (layer "F.Cu") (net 1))
 (arc (start 108.066 124.6475) (mid 107.044 123.6255) (end 106.021999 124.6475) (width 1.751) (layer "F.Cu") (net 1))
 (arc (start 146.902 88.648) (mid 147.924 89.67) (end 148.946 88.648) (width 1.751) (layer "F.Cu") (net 1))
 (arc (start 150.989999 182.552499) (mid 149.968 183.5745) (end 148.946 182.552499) (width 1.751) (layer "F.Cu") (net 1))
 (arc (start 114.198 88.648) (mid 115.219999 89.67) (end 116.242 88.648) (width 1.751) (layer "F.Cu") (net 1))
 (arc (start 103.978 124.439125) (mid 102.955999 123.417125) (end 101.934 124.439125) (width 1.751) (layer "F.Cu") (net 1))
 (arc (start 48.79 174.064575) (mid 47.768 175.086575) (end 46.745999 174.064575) (width 1.751) (layer "F.Cu") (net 1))
 (arc (start 155.078 179.817291) (mid 154.056 180.839291) (end 153.034 179.817291) (width 1.751) (layer "F.Cu") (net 1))
 (arc (start 163.253999 88.647999) (mid 162.355989 90.815989) (end 160.187999 91.713999) (width 1.751) (layer "F.Cu") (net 1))
 (arc (start 162.552499 97.846) (mid 163.574499 98.868) (end 162.552499 99.889999) (width 1.751) (layer "F.Cu") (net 1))
 (arc (start 56.965999 179.817291) (mid 55.944 180.839291) (end 54.922 179.817291) (width 1.751) (layer "F.Cu") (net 1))
 (arc (start 104.129 106.021999) (mid 106.296989 106.92001) (end 107.195 109.088) (width 1.751) (layer "F.Cu") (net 1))
 (arc (start 46.745999 121.351999) (mid 47.64401 119.18401) (end 49.811999 118.285999) (width 1.751) (layer "F.Cu") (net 1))
 (arc (start 83.538 121.351999) (mid 82.515999 120.33) (end 81.494 121.351999) (width 1.751) (layer "F.Cu") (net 1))
 (arc (start 162.552499 114.198) (mid 163.574499 115.219999) (end 162.552499 116.242) (width 1.751) (layer "F.Cu") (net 1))
 (arc (start 91.713999 121.351999) (mid 90.692 120.33) (end 89.67 121.351999) (width 1.751) (layer "F.Cu") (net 1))
 (arc (start 69.23 182.552499) (mid 68.207999 183.5745) (end 67.186 182.552499) (width 1.751) (layer "F.Cu") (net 1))
 (arc (start 106.021999 182.552499) (mid 105 183.5745) (end 103.978 182.552499) (width 1.751) (layer "F.Cu") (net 1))
 (arc (start 114.198 182.552499) (mid 113.176 183.5745) (end 112.154 182.552499) (width 1.751) (layer "F.Cu") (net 1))
 (arc (start 124.418 27.447499) (mid 125.44 26.425499) (end 126.461999 27.447499) (width 1.751) (layer "F.Cu") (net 1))
 (arc (start 63.098 121.351999) (mid 62.076 120.33) (end 61.053999 121.351999) (width 1.751) (layer "F.Cu") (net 1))
 (arc (start 153.034 30.182708) (mid 154.056 29.160708) (end 155.078 30.182708) (width 1.751) (layer "F.Cu") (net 1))
 (arc (start 132.594 27.447499) (mid 133.615999 26.425499) (end 134.638 27.447499) (width 1.751) (layer "F.Cu") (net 1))
 (segment (start 56.965999 88.648) (end 56.965999 30.182708) (width 1.751) (layer "F.Cu") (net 2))
 (segment (start 49.811999 91.713999) (end 101.923 91.713999) (width 1.751) (layer "F.Cu") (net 2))
 (segment (start 47.4475 95.801999) (end 104.129 95.801999) (width 1.751) (layer "F.Cu") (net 2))
 (segment (start 79.449999 27.447499) (end 79.449999 88.648) (width 1.751) (layer "F.Cu") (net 2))
 (segment (start 91.713999 32.461394) (end 91.713999 88.648) (width 1.751) (layer "F.Cu") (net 2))
 (segment (start 85.582 88.648) (end 85.582 27.447499) (width 1.751) (layer "F.Cu") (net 2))
 (segment (start 95.801999 33.6975) (end 95.801999 88.648) (width 1.751) (layer "F.Cu") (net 2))
 (segment (start 50.833999 35.439037) (end 50.833999 88.648) (width 1.751) (layer "F.Cu") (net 2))
 (segment (start 54.922 30.182708) (end 54.922 88.648) (width 1.751) (layer "F.Cu") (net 2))
 (segment (start 67.186 27.447499) (end 67.186 88.648) (width 1.751) (layer "F.Cu") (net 2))
 (segment (start 81.494 88.648) (end 81.494 27.447499) (width 1.751) (layer "F.Cu") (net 2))
 (segment (start 65.141999 88.648) (end 65.141999 27.447499) (width 1.751) (layer "F.Cu") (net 2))
 (segment (start 47.4475 103.978) (end 104.129 103.978) (width 1.751) (layer "F.Cu") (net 2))
 (segment (start 103.978 29.4915) (end 103.978 85.560874) (width 1.751) (layer "F.Cu") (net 2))
 (segment (start 73.318 88.648) (end 73.318 27.447499) (width 1.751) (layer "F.Cu") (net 2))
 (segment (start 52.877999 88.648) (end 52.877999 35.439037) (width 1.751) (layer "F.Cu") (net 2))
 (segment (start 101.934 85.560874) (end 101.934 29.4915) (width 1.751) (layer "F.Cu") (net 2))
 (segment (start 87.625999 27.447499) (end 87.625999 88.648) (width 1.751) (layer "F.Cu") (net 2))
 (segment (start 47.4475 99.889999) (end 104.129 99.889999) (width 1.751) (layer "F.Cu") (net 2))
 (segment (start 71.273999 27.447499) (end 71.273999 88.648) (width 1.751) (layer "F.Cu") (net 2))
 (segment (start 63.098 27.447499) (end 63.098 88.648) (width 1.751) (layer "F.Cu") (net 2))
 (segment (start 107.195 90) (end 107.195 100.912) (width 1.751) (layer "F.Cu") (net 2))
 (segment (start 101.923 93.758) (end 47.4475 93.758) (width 1.751) (layer "F.Cu") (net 2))
 (segment (start 61.053999 88.648) (end 61.053999 27.447499) (width 1.751) (layer "F.Cu") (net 2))
 (segment (start 48.79 88.648) (end 48.79 35.935424) (width 1.751) (layer "F.Cu") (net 2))
 (segment (start 77.406 88.648) (end 77.406 27.447499) (width 1.751) (layer "F.Cu") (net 2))
 (segment (start 46.745999 35.935424) (end 46.745999 88.648) (width 1.751) (layer "F.Cu") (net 2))
 (segment (start 99.889999 29.4915) (end 99.889999 88.648) (width 1.751) (layer "F.Cu") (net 2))
 (segment (start 89.67 88.648) (end 89.67 27.447499) (width 1.751) (layer "F.Cu") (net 2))
 (segment (start 83.538 27.447499) (end 83.538 88.648) (width 1.751) (layer "F.Cu") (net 2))
 (segment (start 69.23 88.648) (end 69.23 27.447499) (width 1.751) (layer "F.Cu") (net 2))
 (segment (start 59.01 27.447499) (end 59.01 88.648) (width 1.751) (layer "F.Cu") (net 2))
 (segment (start 104.129 97.846) (end 47.4475 97.846) (width 1.751) (layer "F.Cu") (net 2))
 (segment (start 93.758 88.648) (end 93.758 32.461394) (width 1.751) (layer "F.Cu") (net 2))
 (segment (start 96.7645 26.425499) (end 100.912 26.425499) (width 1.751) (layer "F.Cu") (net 2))
 (segment (start 104.129 101.934) (end 47.4475 101.934) (width 1.751) (layer "F.Cu") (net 2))
 (segment (start 97.846 88.648) (end 97.846 33.6975) (width 1.751) (layer "F.Cu") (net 2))
 (segment (start 75.362 27.447499) (end 75.362 88.648) (width 1.751) (layer "F.Cu") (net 2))
 (arc (start 61.053999 27.447499) (mid 60.032 26.425499) (end 59.01 27.447499) (width 1.751) (layer "F.Cu") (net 2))
 (arc (start 69.23 27.447499) (mid 68.207999 26.425499) (end 67.186 27.447499) (width 1.751) (layer "F.Cu") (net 2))
 (arc (start 63.098 88.648) (mid 62.076 89.67) (end 61.053999 88.648) (width 1.751) (layer "F.Cu") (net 2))
 (arc (start 73.318 27.447499) (mid 72.295999 26.425499) (end 71.273999 27.447499) (width 1.751) (layer "F.Cu") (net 2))
 (arc (start 47.4475 93.758) (mid 46.425499 94.779999) (end 47.4475 95.801999) (width 1.751) (layer "F.Cu") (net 2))
 (arc (start 67.186 88.648) (mid 66.164 89.67) (end 65.141999 88.648) (width 1.751) (layer "F.Cu") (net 2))
 (arc (start 48.79 35.935424) (mid 47.768 34.913424) (end 46.745999 35.935424) (width 1.751) (layer "F.Cu") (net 2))
 (arc (start 52.877999 35.439037) (mid 51.856 34.417037) (end 50.833999 35.439037) (width 1.751) (layer "F.Cu") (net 2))
 (arc (start 77.406 27.447499) (mid 76.384 26.425499) (end 75.362 27.447499) (width 1.751) (layer "F.Cu") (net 2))
 (arc (start 104.129 99.889999) (mid 105.151 100.912) (end 104.129 101.934) (width 1.751) (layer "F.Cu") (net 2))
 (arc (start 101.934 29.4915) (mid 100.912 28.4695) (end 99.889999 29.4915) (width 1.751) (layer "F.Cu") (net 2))
 (arc (start 47.4475 101.934) (mid 46.425499 102.955999) (end 47.4475 103.978) (width 1.751) (layer "F.Cu") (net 2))
 (arc (start 104.129 95.801999) (mid 105.151 96.824) (end 104.129 97.846) (width 1.751) (layer "F.Cu") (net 2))
 (arc (start 85.582 27.447499) (mid 84.56 26.425499) (end 83.538 27.447499) (width 1.751) (layer "F.Cu") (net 2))
 (arc (start 54.922 88.648) (mid 53.9 89.67) (end 52.877999 88.648) (width 1.751) (layer "F.Cu") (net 2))
 (arc (start 79.449999 88.648) (mid 78.428 89.67) (end 77.406 88.648) (width 1.751) (layer "F.Cu") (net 2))
 (arc (start 47.4475 97.846) (mid 46.425499 98.868) (end 47.4475 99.889999) (width 1.751) (layer "F.Cu") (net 2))
 (arc (start 65.141999 27.447499) (mid 64.119999 26.425499) (end 63.098 27.447499) (width 1.751) (layer "F.Cu") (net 2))
 (arc (start 83.538 88.648) (mid 82.515999 89.67) (end 81.494 88.648) (width 1.751) (layer "F.Cu") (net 2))
 (arc (start 103.978 85.560874) (mid 102.955999 86.582874) (end 101.934 85.560874) (width 1.751) (layer "F.Cu") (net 2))
 (arc (start 87.625999 88.648) (mid 86.604 89.67) (end 85.582 88.648) (width 1.751) (layer "F.Cu") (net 2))
 (arc (start 81.494 27.447499) (mid 80.472 26.425499) (end 79.449999 27.447499) (width 1.751) (layer "F.Cu") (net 2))
 (arc (start 91.713999 88.648) (mid 90.692 89.67) (end 89.67 88.648) (width 1.751) (layer "F.Cu") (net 2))
 (arc (start 89.67 27.447499) (mid 88.648 26.425499) (end 87.625999 27.447499) (width 1.751) (layer "F.Cu") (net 2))
 (arc (start 56.965999 30.182708) (mid 55.944 29.160708) (end 54.922 30.182708) (width 1.751) (layer "F.Cu") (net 2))
 (arc (start 99.889999 88.648) (mid 98.868 89.67) (end 97.846 88.648) (width 1.751) (layer "F.Cu") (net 2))
 (arc (start 50.833999 88.648) (mid 49.812 89.67) (end 48.79 88.648) (width 1.751) (layer "F.Cu") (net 2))
 (arc (start 100.912 26.425499) (mid 103.079989 27.32351) (end 103.978 29.4915) (width 1.751) (layer "F.Cu") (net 2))
 (arc (start 75.362 88.648) (mid 74.34 89.67) (end 73.318 88.648) (width 1.751) (layer "F.Cu") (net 2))
 (arc (start 59.01 88.648) (mid 57.988 89.67) (end 56.965999 88.648) (width 1.751) (layer "F.Cu") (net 2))
 (arc (start 101.923 91.713999) (mid 102.945 92.736) (end 101.923 93.758) (width 1.751) (layer "F.Cu") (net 2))
 (arc (start 49.811999 91.713999) (mid 47.64401 90.815989) (end 46.745999 88.648) (width 1.751) (layer "F.Cu") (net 2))
 (arc (start 95.801999 88.648) (mid 94.779999 89.67) (end 93.758 88.648) (width 1.751) (layer "F.Cu") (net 2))
 (arc (start 71.273999 88.648) (mid 70.252 89.67) (end 69.23 88.648) (width 1.751) (layer "F.Cu") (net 2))
 (arc (start 97.846 33.6975) (mid 96.824 32.6755) (end 95.801999 33.6975) (width 1.751) (layer "F.Cu") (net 2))
 (arc (start 93.758 32.461394) (mid 92.736 31.439394) (end 91.713999 32.461394) (width 1.751) (layer "F.Cu") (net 2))
 (arc (start 107.195 100.912) (mid 106.296989 103.079989) (end 104.129 103.978) (width 1.751) (layer "F.Cu") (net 2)))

